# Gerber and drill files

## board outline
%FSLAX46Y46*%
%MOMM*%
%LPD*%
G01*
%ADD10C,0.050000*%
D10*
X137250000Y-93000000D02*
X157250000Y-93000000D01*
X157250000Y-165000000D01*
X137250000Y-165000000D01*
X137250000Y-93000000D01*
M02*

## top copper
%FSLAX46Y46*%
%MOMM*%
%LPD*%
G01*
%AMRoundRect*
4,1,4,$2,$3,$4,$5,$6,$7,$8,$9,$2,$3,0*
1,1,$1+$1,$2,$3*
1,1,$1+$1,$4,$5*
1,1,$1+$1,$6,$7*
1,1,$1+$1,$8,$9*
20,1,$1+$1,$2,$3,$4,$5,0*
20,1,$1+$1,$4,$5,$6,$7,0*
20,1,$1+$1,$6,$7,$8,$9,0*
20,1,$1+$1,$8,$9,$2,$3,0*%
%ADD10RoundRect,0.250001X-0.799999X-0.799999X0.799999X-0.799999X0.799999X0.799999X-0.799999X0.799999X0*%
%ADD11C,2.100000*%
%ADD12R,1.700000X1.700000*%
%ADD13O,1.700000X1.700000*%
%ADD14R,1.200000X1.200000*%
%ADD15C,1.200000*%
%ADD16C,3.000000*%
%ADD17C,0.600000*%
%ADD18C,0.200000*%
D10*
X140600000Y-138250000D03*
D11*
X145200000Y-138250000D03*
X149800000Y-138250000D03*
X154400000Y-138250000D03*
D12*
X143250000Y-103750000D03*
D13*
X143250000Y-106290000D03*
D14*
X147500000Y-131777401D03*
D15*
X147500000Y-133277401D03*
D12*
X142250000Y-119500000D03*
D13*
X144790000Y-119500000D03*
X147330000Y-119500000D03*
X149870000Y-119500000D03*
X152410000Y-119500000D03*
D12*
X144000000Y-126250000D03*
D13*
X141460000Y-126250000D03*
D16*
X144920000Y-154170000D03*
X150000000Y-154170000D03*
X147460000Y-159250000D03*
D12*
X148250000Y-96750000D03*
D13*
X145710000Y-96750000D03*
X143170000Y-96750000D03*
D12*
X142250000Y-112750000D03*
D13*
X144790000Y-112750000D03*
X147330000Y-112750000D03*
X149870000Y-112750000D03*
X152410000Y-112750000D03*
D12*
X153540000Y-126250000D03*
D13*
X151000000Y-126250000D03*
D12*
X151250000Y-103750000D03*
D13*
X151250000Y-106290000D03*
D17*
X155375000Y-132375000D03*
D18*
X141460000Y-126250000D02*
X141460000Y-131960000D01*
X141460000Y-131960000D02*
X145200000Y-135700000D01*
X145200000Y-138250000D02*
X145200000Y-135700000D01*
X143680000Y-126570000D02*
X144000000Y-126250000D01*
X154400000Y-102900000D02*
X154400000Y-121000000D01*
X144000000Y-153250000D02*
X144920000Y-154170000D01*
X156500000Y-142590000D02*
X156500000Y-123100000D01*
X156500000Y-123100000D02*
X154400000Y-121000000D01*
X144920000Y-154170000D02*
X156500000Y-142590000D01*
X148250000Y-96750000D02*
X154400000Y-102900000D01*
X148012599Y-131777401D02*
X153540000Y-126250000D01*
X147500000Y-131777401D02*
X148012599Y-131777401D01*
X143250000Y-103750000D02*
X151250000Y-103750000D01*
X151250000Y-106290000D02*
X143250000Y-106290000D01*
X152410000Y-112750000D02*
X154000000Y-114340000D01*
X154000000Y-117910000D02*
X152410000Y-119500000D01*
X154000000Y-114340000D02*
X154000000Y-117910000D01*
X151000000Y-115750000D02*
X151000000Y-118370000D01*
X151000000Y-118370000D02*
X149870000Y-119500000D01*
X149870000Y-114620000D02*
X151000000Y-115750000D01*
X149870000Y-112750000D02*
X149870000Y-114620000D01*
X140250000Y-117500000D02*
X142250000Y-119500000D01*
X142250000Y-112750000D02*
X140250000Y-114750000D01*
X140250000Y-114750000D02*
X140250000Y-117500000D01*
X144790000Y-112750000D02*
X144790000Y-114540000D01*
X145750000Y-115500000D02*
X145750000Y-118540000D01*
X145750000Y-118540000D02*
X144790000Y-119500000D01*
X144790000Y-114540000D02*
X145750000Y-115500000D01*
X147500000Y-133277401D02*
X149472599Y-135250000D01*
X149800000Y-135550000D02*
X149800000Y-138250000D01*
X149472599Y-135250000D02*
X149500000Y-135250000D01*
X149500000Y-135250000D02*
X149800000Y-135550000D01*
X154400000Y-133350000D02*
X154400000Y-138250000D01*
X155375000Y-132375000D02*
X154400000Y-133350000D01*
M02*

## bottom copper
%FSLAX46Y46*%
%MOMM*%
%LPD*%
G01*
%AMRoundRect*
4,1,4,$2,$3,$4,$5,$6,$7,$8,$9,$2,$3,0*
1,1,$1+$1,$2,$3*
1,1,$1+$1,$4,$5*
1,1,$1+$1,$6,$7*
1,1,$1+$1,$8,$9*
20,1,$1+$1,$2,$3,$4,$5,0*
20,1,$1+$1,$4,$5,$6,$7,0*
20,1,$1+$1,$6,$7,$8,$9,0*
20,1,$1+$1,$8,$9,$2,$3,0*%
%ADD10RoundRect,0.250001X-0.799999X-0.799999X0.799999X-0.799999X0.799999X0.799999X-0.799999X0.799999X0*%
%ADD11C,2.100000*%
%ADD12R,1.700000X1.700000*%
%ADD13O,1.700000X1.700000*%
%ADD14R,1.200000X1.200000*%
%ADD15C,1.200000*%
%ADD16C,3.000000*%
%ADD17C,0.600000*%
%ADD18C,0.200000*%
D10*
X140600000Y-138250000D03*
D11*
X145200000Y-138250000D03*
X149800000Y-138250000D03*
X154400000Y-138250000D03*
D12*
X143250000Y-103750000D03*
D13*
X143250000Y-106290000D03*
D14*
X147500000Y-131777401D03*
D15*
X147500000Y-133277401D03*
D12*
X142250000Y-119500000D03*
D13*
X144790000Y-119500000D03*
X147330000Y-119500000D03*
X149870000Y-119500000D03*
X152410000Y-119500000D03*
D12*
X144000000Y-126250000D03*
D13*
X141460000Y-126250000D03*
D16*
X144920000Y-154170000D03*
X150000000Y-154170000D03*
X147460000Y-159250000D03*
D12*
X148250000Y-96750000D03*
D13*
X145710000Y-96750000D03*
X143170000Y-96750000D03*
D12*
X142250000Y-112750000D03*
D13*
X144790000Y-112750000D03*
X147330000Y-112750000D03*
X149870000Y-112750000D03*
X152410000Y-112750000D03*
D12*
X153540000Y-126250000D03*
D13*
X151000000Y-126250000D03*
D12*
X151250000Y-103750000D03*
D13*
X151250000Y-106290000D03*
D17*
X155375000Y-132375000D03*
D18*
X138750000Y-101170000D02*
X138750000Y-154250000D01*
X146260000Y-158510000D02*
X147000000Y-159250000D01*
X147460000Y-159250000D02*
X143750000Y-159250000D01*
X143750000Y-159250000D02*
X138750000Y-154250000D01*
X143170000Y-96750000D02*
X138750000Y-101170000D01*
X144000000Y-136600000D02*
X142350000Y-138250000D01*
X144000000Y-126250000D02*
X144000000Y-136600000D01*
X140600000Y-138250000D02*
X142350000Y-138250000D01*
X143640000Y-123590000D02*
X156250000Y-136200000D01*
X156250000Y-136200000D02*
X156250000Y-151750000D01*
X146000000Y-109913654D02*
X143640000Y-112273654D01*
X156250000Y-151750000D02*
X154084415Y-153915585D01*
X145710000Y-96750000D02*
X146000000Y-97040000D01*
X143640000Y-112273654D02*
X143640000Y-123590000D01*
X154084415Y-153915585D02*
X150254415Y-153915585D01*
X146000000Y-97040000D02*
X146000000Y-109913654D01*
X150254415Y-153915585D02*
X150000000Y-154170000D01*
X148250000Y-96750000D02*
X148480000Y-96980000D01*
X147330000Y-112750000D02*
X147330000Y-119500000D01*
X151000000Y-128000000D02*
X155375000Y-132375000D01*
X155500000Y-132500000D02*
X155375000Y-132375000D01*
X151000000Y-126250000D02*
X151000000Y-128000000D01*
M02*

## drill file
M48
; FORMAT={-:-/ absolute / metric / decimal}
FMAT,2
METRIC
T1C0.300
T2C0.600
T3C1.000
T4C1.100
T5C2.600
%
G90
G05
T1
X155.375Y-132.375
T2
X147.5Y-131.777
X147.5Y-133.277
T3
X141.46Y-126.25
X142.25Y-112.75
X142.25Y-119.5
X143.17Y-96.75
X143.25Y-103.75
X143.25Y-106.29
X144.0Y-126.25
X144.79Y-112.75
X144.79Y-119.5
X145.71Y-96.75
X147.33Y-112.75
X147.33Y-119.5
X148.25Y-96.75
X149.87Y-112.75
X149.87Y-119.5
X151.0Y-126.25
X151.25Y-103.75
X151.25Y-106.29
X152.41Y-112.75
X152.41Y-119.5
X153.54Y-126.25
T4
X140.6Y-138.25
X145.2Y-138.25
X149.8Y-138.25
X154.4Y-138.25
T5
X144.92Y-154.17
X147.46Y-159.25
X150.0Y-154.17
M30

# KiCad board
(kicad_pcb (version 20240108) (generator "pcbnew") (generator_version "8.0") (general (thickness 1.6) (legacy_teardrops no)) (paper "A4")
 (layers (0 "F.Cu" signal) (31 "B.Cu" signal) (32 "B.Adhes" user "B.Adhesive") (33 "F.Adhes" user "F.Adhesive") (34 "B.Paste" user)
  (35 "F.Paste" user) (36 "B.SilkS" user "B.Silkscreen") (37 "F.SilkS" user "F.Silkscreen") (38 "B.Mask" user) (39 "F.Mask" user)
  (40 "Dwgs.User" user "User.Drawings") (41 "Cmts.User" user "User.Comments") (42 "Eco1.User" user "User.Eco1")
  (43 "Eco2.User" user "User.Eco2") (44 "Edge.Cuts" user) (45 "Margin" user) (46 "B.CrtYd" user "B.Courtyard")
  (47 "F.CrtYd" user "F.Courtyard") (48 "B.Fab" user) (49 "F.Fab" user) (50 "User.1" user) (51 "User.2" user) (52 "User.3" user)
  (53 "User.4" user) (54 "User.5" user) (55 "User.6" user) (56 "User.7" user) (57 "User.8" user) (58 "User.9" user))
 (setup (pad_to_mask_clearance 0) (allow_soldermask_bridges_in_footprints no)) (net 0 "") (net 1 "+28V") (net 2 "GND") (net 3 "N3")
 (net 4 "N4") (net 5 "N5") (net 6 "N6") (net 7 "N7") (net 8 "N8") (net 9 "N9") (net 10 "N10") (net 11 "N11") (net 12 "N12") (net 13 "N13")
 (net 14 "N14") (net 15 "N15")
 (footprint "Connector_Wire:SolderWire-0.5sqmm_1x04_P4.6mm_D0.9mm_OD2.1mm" (layer "F.Cu") (at 140.6 138.25)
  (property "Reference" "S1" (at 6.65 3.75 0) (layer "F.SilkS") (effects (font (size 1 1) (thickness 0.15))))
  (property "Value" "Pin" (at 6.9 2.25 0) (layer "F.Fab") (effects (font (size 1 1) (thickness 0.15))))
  (pad "1" thru_hole roundrect (at 0 0) (size 2.1 2.1) (drill 1.1) (layers "*.Cu" "*.Mask") (remove_unused_layers no)
   (roundrect_rratio 0.119048) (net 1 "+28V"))
  (pad "2" thru_hole circle (at 4.6 0) (size 2.1 2.1) (drill 1.1) (layers "*.Cu" "*.Mask") (remove_unused_layers no) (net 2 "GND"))
  (pad "3" thru_hole circle (at 9.2 0) (size 2.1 2.1) (drill 1.1) (layers "*.Cu" "*.Mask") (remove_unused_layers no) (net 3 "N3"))
  (pad "4" thru_hole circle (at 13.8 0) (size 2.1 2.1) (drill 1.1) (layers "*.Cu" "*.Mask") (remove_unused_layers no) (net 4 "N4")))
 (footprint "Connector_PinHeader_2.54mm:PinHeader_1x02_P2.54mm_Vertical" (layer "F.Cu") (at 143.25 103.75)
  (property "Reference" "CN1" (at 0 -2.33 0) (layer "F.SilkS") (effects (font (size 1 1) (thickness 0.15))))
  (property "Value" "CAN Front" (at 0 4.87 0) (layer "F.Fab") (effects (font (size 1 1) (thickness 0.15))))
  (pad "1" thru_hole rect (at 0 0) (size 1.7 1.7) (drill 1) (layers "*.Cu" "*.Mask") (remove_unused_layers no) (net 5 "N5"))
  (pad "2" thru_hole oval (at 0 2.54) (size 1.7 1.7) (drill 1) (layers "*.Cu" "*.Mask") (remove_unused_layers no) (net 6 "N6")))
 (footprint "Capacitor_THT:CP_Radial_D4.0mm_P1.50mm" (layer "F.Cu") (at 147.5 131.777401 -90)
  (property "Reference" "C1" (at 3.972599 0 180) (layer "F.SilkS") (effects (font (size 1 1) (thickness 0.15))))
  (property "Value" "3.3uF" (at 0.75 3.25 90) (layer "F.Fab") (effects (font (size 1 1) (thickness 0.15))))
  (pad "1" thru_hole rect (at 0 0 270) (size 1.2 1.2) (drill 0.6) (layers "*.Cu" "*.Mask") (remove_unused_layers no) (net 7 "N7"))
  (pad "2" thru_hole circle (at 1.5 0 270) (size 1.2 1.2) (drill 0.6) (layers "*.Cu" "*.Mask") (remove_unused_layers no) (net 3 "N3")))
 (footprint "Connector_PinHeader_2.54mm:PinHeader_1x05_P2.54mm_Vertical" (layer "F.Cu") (at 142.25 119.5 90)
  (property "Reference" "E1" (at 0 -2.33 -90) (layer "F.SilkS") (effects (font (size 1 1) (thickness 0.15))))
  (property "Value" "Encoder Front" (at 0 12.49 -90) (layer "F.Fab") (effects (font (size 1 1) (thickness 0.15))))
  (pad "1" thru_hole rect (at 0 0 90) (size 1.7 1.7) (drill 1) (layers "*.Cu" "*.Mask") (remove_unused_layers no) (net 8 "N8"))
  (pad "2" thru_hole oval (at 0 2.54 90) (size 1.7 1.7) (drill 1) (layers "*.Cu" "*.Mask") (remove_unused_layers no) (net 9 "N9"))
  (pad "3" thru_hole oval (at 0 5.08 90) (size 1.7 1.7) (drill 1) (layers "*.Cu" "*.Mask") (remove_unused_layers no) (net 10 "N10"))
  (pad "4" thru_hole oval (at 0 7.62 90) (size 1.7 1.7) (drill 1) (layers "*.Cu" "*.Mask") (remove_unused_layers no) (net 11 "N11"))
  (pad "5" thru_hole oval (at 0 10.16 90) (size 1.7 1.7) (drill 1) (layers "*.Cu" "*.Mask") (remove_unused_layers no) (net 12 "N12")))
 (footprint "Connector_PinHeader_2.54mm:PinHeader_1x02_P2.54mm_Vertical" (layer "F.Cu") (at 144 126.25 -90)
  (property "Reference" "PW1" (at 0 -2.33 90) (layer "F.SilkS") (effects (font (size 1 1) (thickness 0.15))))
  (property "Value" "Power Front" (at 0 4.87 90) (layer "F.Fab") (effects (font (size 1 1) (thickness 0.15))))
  (pad "1" thru_hole rect (at 0 0 270) (size 1.7 1.7) (drill 1) (layers "*.Cu" "*.Mask") (remove_unused_layers no) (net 1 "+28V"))
  (pad "2" thru_hole oval (at 0 2.54 270) (size 1.7 1.7) (drill 1) (layers "*.Cu" "*.Mask") (remove_unused_layers no) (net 2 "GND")))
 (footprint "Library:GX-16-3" (layer "F.Cu") (at 147.46 156.71)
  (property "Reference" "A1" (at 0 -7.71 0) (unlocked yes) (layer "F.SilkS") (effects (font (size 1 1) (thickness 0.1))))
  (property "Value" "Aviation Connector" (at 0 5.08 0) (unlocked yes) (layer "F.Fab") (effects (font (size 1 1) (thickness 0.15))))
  (pad "1" thru_hole circle (at -2.54 -2.54) (size 3 3) (drill 2.6) (layers "*.Cu" "*.Mask") (remove_unused_layers no) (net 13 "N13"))
  (pad "2" thru_hole circle (at 2.54 -2.54) (size 3 3) (drill 2.6) (layers "*.Cu" "*.Mask") (remove_unused_layers no) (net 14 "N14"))
  (pad "3" thru_hole circle (at 0 2.54) (size 3 3) (drill 2.6) (layers "*.Cu" "*.Mask") (remove_unused_layers no) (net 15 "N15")))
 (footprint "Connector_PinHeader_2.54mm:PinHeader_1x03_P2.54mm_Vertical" (layer "B.Cu") (at 148.25 96.75 90)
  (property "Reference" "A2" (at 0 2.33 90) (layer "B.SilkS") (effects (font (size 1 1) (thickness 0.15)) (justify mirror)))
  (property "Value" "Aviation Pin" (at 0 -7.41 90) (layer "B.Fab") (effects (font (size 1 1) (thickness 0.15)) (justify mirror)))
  (pad "1" thru_hole rect (at 0 0 90) (size 1.7 1.7) (drill 1) (layers "*.Cu" "*.Mask") (remove_unused_layers no) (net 13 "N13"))
  (pad "2" thru_hole oval (at 0 -2.54 90) (size 1.7 1.7) (drill 1) (layers "*.Cu" "*.Mask") (remove_unused_layers no) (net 14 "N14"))
  (pad "3" thru_hole oval (at 0 -5.08 90) (size 1.7 1.7) (drill 1) (layers "*.Cu" "*.Mask") (remove_unused_layers no) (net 15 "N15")))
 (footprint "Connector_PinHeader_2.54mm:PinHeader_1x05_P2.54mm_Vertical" (layer "B.Cu") (at 142.25 112.75 -90)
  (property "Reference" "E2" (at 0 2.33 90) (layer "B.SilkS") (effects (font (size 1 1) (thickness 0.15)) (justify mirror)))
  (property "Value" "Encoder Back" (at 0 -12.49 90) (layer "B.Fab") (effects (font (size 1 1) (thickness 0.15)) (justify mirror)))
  (pad "1" thru_hole rect (at 0 0 270) (size 1.7 1.7) (drill 1) (layers "*.Cu" "*.Mask") (remove_unused_layers no) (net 8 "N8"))
  (pad "2" thru_hole oval (at 0 -2.54 270) (size 1.7 1.7) (drill 1) (layers "*.Cu" "*.Mask") (remove_unused_layers no) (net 9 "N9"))
  (pad "3" thru_hole oval (at 0 -5.08 270) (size 1.7 1.7) (drill 1) (layers "*.Cu" "*.Mask") (remove_unused_layers no) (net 10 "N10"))
  (pad "4" thru_hole oval (at 0 -7.62 270) (size 1.7 1.7) (drill 1) (layers "*.Cu" "*.Mask") (remove_unused_layers no) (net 11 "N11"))
  (pad "5" thru_hole oval (at 0 -10.16 270) (size 1.7 1.7) (drill 1) (layers "*.Cu" "*.Mask") (remove_unused_layers no) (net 12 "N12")))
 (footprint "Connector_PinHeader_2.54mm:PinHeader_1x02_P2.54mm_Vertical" (layer "B.Cu") (at 153.54 126.25 90)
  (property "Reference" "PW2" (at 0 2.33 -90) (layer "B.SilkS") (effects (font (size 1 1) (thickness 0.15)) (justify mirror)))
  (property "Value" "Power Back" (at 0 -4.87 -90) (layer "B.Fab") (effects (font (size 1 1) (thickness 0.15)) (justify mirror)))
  (pad "1" thru_hole rect (at 0 0 90) (size 1.7 1.7) (drill 1) (layers "*.Cu" "*.Mask") (remove_unused_layers no) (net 7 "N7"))
  (pad "2" thru_hole oval (at 0 -2.54 90) (size 1.7 1.7) (drill 1) (layers "*.Cu" "*.Mask") (remove_unused_layers no) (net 4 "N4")))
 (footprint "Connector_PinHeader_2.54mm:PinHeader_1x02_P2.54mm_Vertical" (layer "B.Cu") (at 151.25 103.75 180)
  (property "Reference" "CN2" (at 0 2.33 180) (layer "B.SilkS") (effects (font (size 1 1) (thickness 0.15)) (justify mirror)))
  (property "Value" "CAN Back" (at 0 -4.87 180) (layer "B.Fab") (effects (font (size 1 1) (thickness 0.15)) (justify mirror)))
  (pad "1" thru_hole rect (at 0 0 180) (size 1.7 1.7) (drill 1) (layers "*.Cu" "*.Mask") (remove_unused_layers no) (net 5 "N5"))
  (pad "2" thru_hole oval (at 0 -2.54 180) (size 1.7 1.7) (drill 1) (layers "*.Cu" "*.Mask") (remove_unused_layers no) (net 6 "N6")))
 (gr_rect (start 137.25 93) (end 157.25 165) (stroke (width 0.05) (type default)) (fill none) (layer "Edge.Cuts"))
 (segment (start 138.75 101.17) (end 138.75 154.25) (width 0.2) (layer "B.Cu") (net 15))
 (segment (start 146.26 158.51) (end 147 159.25) (width 0.2) (layer "B.Cu") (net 15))
 (segment (start 147.46 159.25) (end 143.75 159.25) (width 0.2) (layer "B.Cu") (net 15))
 (segment (start 143.75 159.25) (end 138.75 154.25) (width 0.2) (layer "B.Cu") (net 15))
 (segment (start 143.17 96.75) (end 138.75 101.17) (width 0.2) (layer "B.Cu") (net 15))
 (segment (start 141.46 126.25) (end 141.46 131.96) (width 0.2) (layer "F.Cu") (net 2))
 (segment (start 141.46 131.96) (end 145.2 135.7) (width 0.2) (layer "F.Cu") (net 2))
 (segment (start 145.2 138.25) (end 145.2 135.7) (width 0.2) (layer "F.Cu") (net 2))
 (segment (start 143.68 126.57) (end 144 126.25) (width 0.2) (layer "F.Cu") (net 1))
 (segment (start 144 136.6) (end 142.35 138.25) (width 0.2) (layer "B.Cu") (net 1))
 (segment (start 144 126.25) (end 144 136.6) (width 0.2) (layer "B.Cu") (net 1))
 (segment (start 140.6 138.25) (end 142.35 138.25) (width 0.2) (layer "B.Cu") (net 1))
 (segment (start 143.64 123.59) (end 156.25 136.2) (width 0.2) (layer "B.Cu") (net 14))
 (segment (start 156.25 136.2) (end 156.25 151.75) (width 0.2) (layer "B.Cu") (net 14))
 (segment (start 146 109.913654) (end 143.64 112.273654) (width 0.2) (layer "B.Cu") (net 14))
 (segment (start 156.25 151.75) (end 154.084415 153.915585) (width 0.2) (layer "B.Cu") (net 14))
 (segment (start 145.71 96.75) (end 146 97.04) (width 0.2) (layer "B.Cu") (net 14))
 (segment (start 143.64 112.273654) (end 143.64 123.59) (width 0.2) (layer "B.Cu") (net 14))
 (segment (start 154.084415 153.915585) (end 150.254415 153.915585) (width 0.2) (layer "B.Cu") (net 14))
 (segment (start 146 97.04) (end 146 109.913654) (width 0.2) (layer "B.Cu") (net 14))
 (segment (start 150.254415 153.915585) (end 150 154.17) (width 0.2) (layer "B.Cu") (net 14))
 (segment (start 154.4 102.9) (end 154.4 121) (width 0.2) (layer "F.Cu") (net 13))
 (segment (start 144 153.25) (end 144.92 154.17) (width 0.2) (layer "F.Cu") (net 13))
 (segment (start 156.5 142.59) (end 156.5 123.1) (width 0.2) (layer "F.Cu") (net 13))
 (segment (start 156.5 123.1) (end 154.4 121) (width 0.2) (layer "F.Cu") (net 13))
 (segment (start 144.92 154.17) (end 156.5 142.59) (width 0.2) (layer "F.Cu") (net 13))
 (segment (start 148.25 96.75) (end 154.4 102.9) (width 0.2) (layer "F.Cu") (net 13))
 (segment (start 148.25 96.75) (end 148.48 96.98) (width 0.2) (layer "B.Cu") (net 13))
 (segment (start 148.012599 131.777401) (end 153.54 126.25) (width 0.2) (layer "F.Cu") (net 7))
 (segment (start 147.5 131.777401) (end 148.012599 131.777401) (width 0.2) (layer "F.Cu") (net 7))
 (segment (start 143.25 103.75) (end 151.25 103.75) (width 0.2) (layer "F.Cu") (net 5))
 (segment (start 151.25 106.29) (end 143.25 106.29) (width 0.2) (layer "F.Cu") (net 6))
 (segment (start 152.41 112.75) (end 154 114.34) (width 0.2) (layer "F.Cu") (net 12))
 (segment (start 154 117.91) (end 152.41 119.5) (width 0.2) (layer "F.Cu") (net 12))
 (segment (start 154 114.34) (end 154 117.91) (width 0.2) (layer "F.Cu") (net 12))
 (segment (start 151 115.75) (end 151 118.37) (width 0.2) (layer "F.Cu") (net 11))
 (segment (start 151 118.37) (end 149.87 119.5) (width 0.2) (layer "F.Cu") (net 11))
 (segment (start 149.87 114.62) (end 151 115.75) (width 0.2) (layer "F.Cu") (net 11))
 (segment (start 149.87 112.75) (end 149.87 114.62) (width 0.2) (layer "F.Cu") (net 11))
 (segment (start 140.25 117.5) (end 142.25 119.5) (width 0.2) (layer "F.Cu") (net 8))
 (segment (start 142.25 112.75) (end 140.25 114.75) (width 0.2) (layer "F.Cu") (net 8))
 (segment (start 140.25 114.75) (end 140.25 117.5) (width 0.2) (layer "F.Cu") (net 8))
 (segment (start 147.33 112.75) (end 147.33 119.5) (width 0.2) (layer "B.Cu") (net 10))
 (segment (start 144.79 112.75) (end 144.79 114.54) (width 0.2) (layer "F.Cu") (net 9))
 (segment (start 145.75 115.5) (end 145.75 118.54) (width 0.2) (layer "F.Cu") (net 9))
 (segment (start 145.75 118.54) (end 144.79 119.5) (width 0.2) (layer "F.Cu") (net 9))
 (segment (start 144.79 114.54) (end 145.75 115.5) (width 0.2) (layer "F.Cu") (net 9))
 (segment (start 147.5 133.277401) (end 149.472599 135.25) (width 0.2) (layer "F.Cu") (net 3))
 (segment (start 149.8 135.55) (end 149.8 138.25) (width 0.2) (layer "F.Cu") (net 3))
 (segment (start 149.472599 135.25) (end 149.5 135.25) (width 0.2) (layer "F.Cu") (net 3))
 (segment (start 149.5 135.25) (end 149.8 135.55) (width 0.2) (layer "F.Cu") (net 3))
 (segment (start 154.4 133.35) (end 154.4 138.25) (width 0.2) (layer "F.Cu") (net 4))
 (segment (start 155.375 132.375) (end 154.4 133.35) (width 0.2) (layer "F.Cu") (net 4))
 (via (at 155.375 132.375) (size 0.6) (drill 0.3) (layers "F.Cu" "B.Cu") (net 4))
 (segment (start 151 128) (end 155.375 132.375) (width 0.2) (layer "B.Cu") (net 4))
 (segment (start 155.5 132.5) (end 155.375 132.375) (width 0.2) (layer "B.Cu") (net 4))
 (segment (start 151 126.25) (end 151 128) (width 0.2) (layer "B.Cu") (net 4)))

